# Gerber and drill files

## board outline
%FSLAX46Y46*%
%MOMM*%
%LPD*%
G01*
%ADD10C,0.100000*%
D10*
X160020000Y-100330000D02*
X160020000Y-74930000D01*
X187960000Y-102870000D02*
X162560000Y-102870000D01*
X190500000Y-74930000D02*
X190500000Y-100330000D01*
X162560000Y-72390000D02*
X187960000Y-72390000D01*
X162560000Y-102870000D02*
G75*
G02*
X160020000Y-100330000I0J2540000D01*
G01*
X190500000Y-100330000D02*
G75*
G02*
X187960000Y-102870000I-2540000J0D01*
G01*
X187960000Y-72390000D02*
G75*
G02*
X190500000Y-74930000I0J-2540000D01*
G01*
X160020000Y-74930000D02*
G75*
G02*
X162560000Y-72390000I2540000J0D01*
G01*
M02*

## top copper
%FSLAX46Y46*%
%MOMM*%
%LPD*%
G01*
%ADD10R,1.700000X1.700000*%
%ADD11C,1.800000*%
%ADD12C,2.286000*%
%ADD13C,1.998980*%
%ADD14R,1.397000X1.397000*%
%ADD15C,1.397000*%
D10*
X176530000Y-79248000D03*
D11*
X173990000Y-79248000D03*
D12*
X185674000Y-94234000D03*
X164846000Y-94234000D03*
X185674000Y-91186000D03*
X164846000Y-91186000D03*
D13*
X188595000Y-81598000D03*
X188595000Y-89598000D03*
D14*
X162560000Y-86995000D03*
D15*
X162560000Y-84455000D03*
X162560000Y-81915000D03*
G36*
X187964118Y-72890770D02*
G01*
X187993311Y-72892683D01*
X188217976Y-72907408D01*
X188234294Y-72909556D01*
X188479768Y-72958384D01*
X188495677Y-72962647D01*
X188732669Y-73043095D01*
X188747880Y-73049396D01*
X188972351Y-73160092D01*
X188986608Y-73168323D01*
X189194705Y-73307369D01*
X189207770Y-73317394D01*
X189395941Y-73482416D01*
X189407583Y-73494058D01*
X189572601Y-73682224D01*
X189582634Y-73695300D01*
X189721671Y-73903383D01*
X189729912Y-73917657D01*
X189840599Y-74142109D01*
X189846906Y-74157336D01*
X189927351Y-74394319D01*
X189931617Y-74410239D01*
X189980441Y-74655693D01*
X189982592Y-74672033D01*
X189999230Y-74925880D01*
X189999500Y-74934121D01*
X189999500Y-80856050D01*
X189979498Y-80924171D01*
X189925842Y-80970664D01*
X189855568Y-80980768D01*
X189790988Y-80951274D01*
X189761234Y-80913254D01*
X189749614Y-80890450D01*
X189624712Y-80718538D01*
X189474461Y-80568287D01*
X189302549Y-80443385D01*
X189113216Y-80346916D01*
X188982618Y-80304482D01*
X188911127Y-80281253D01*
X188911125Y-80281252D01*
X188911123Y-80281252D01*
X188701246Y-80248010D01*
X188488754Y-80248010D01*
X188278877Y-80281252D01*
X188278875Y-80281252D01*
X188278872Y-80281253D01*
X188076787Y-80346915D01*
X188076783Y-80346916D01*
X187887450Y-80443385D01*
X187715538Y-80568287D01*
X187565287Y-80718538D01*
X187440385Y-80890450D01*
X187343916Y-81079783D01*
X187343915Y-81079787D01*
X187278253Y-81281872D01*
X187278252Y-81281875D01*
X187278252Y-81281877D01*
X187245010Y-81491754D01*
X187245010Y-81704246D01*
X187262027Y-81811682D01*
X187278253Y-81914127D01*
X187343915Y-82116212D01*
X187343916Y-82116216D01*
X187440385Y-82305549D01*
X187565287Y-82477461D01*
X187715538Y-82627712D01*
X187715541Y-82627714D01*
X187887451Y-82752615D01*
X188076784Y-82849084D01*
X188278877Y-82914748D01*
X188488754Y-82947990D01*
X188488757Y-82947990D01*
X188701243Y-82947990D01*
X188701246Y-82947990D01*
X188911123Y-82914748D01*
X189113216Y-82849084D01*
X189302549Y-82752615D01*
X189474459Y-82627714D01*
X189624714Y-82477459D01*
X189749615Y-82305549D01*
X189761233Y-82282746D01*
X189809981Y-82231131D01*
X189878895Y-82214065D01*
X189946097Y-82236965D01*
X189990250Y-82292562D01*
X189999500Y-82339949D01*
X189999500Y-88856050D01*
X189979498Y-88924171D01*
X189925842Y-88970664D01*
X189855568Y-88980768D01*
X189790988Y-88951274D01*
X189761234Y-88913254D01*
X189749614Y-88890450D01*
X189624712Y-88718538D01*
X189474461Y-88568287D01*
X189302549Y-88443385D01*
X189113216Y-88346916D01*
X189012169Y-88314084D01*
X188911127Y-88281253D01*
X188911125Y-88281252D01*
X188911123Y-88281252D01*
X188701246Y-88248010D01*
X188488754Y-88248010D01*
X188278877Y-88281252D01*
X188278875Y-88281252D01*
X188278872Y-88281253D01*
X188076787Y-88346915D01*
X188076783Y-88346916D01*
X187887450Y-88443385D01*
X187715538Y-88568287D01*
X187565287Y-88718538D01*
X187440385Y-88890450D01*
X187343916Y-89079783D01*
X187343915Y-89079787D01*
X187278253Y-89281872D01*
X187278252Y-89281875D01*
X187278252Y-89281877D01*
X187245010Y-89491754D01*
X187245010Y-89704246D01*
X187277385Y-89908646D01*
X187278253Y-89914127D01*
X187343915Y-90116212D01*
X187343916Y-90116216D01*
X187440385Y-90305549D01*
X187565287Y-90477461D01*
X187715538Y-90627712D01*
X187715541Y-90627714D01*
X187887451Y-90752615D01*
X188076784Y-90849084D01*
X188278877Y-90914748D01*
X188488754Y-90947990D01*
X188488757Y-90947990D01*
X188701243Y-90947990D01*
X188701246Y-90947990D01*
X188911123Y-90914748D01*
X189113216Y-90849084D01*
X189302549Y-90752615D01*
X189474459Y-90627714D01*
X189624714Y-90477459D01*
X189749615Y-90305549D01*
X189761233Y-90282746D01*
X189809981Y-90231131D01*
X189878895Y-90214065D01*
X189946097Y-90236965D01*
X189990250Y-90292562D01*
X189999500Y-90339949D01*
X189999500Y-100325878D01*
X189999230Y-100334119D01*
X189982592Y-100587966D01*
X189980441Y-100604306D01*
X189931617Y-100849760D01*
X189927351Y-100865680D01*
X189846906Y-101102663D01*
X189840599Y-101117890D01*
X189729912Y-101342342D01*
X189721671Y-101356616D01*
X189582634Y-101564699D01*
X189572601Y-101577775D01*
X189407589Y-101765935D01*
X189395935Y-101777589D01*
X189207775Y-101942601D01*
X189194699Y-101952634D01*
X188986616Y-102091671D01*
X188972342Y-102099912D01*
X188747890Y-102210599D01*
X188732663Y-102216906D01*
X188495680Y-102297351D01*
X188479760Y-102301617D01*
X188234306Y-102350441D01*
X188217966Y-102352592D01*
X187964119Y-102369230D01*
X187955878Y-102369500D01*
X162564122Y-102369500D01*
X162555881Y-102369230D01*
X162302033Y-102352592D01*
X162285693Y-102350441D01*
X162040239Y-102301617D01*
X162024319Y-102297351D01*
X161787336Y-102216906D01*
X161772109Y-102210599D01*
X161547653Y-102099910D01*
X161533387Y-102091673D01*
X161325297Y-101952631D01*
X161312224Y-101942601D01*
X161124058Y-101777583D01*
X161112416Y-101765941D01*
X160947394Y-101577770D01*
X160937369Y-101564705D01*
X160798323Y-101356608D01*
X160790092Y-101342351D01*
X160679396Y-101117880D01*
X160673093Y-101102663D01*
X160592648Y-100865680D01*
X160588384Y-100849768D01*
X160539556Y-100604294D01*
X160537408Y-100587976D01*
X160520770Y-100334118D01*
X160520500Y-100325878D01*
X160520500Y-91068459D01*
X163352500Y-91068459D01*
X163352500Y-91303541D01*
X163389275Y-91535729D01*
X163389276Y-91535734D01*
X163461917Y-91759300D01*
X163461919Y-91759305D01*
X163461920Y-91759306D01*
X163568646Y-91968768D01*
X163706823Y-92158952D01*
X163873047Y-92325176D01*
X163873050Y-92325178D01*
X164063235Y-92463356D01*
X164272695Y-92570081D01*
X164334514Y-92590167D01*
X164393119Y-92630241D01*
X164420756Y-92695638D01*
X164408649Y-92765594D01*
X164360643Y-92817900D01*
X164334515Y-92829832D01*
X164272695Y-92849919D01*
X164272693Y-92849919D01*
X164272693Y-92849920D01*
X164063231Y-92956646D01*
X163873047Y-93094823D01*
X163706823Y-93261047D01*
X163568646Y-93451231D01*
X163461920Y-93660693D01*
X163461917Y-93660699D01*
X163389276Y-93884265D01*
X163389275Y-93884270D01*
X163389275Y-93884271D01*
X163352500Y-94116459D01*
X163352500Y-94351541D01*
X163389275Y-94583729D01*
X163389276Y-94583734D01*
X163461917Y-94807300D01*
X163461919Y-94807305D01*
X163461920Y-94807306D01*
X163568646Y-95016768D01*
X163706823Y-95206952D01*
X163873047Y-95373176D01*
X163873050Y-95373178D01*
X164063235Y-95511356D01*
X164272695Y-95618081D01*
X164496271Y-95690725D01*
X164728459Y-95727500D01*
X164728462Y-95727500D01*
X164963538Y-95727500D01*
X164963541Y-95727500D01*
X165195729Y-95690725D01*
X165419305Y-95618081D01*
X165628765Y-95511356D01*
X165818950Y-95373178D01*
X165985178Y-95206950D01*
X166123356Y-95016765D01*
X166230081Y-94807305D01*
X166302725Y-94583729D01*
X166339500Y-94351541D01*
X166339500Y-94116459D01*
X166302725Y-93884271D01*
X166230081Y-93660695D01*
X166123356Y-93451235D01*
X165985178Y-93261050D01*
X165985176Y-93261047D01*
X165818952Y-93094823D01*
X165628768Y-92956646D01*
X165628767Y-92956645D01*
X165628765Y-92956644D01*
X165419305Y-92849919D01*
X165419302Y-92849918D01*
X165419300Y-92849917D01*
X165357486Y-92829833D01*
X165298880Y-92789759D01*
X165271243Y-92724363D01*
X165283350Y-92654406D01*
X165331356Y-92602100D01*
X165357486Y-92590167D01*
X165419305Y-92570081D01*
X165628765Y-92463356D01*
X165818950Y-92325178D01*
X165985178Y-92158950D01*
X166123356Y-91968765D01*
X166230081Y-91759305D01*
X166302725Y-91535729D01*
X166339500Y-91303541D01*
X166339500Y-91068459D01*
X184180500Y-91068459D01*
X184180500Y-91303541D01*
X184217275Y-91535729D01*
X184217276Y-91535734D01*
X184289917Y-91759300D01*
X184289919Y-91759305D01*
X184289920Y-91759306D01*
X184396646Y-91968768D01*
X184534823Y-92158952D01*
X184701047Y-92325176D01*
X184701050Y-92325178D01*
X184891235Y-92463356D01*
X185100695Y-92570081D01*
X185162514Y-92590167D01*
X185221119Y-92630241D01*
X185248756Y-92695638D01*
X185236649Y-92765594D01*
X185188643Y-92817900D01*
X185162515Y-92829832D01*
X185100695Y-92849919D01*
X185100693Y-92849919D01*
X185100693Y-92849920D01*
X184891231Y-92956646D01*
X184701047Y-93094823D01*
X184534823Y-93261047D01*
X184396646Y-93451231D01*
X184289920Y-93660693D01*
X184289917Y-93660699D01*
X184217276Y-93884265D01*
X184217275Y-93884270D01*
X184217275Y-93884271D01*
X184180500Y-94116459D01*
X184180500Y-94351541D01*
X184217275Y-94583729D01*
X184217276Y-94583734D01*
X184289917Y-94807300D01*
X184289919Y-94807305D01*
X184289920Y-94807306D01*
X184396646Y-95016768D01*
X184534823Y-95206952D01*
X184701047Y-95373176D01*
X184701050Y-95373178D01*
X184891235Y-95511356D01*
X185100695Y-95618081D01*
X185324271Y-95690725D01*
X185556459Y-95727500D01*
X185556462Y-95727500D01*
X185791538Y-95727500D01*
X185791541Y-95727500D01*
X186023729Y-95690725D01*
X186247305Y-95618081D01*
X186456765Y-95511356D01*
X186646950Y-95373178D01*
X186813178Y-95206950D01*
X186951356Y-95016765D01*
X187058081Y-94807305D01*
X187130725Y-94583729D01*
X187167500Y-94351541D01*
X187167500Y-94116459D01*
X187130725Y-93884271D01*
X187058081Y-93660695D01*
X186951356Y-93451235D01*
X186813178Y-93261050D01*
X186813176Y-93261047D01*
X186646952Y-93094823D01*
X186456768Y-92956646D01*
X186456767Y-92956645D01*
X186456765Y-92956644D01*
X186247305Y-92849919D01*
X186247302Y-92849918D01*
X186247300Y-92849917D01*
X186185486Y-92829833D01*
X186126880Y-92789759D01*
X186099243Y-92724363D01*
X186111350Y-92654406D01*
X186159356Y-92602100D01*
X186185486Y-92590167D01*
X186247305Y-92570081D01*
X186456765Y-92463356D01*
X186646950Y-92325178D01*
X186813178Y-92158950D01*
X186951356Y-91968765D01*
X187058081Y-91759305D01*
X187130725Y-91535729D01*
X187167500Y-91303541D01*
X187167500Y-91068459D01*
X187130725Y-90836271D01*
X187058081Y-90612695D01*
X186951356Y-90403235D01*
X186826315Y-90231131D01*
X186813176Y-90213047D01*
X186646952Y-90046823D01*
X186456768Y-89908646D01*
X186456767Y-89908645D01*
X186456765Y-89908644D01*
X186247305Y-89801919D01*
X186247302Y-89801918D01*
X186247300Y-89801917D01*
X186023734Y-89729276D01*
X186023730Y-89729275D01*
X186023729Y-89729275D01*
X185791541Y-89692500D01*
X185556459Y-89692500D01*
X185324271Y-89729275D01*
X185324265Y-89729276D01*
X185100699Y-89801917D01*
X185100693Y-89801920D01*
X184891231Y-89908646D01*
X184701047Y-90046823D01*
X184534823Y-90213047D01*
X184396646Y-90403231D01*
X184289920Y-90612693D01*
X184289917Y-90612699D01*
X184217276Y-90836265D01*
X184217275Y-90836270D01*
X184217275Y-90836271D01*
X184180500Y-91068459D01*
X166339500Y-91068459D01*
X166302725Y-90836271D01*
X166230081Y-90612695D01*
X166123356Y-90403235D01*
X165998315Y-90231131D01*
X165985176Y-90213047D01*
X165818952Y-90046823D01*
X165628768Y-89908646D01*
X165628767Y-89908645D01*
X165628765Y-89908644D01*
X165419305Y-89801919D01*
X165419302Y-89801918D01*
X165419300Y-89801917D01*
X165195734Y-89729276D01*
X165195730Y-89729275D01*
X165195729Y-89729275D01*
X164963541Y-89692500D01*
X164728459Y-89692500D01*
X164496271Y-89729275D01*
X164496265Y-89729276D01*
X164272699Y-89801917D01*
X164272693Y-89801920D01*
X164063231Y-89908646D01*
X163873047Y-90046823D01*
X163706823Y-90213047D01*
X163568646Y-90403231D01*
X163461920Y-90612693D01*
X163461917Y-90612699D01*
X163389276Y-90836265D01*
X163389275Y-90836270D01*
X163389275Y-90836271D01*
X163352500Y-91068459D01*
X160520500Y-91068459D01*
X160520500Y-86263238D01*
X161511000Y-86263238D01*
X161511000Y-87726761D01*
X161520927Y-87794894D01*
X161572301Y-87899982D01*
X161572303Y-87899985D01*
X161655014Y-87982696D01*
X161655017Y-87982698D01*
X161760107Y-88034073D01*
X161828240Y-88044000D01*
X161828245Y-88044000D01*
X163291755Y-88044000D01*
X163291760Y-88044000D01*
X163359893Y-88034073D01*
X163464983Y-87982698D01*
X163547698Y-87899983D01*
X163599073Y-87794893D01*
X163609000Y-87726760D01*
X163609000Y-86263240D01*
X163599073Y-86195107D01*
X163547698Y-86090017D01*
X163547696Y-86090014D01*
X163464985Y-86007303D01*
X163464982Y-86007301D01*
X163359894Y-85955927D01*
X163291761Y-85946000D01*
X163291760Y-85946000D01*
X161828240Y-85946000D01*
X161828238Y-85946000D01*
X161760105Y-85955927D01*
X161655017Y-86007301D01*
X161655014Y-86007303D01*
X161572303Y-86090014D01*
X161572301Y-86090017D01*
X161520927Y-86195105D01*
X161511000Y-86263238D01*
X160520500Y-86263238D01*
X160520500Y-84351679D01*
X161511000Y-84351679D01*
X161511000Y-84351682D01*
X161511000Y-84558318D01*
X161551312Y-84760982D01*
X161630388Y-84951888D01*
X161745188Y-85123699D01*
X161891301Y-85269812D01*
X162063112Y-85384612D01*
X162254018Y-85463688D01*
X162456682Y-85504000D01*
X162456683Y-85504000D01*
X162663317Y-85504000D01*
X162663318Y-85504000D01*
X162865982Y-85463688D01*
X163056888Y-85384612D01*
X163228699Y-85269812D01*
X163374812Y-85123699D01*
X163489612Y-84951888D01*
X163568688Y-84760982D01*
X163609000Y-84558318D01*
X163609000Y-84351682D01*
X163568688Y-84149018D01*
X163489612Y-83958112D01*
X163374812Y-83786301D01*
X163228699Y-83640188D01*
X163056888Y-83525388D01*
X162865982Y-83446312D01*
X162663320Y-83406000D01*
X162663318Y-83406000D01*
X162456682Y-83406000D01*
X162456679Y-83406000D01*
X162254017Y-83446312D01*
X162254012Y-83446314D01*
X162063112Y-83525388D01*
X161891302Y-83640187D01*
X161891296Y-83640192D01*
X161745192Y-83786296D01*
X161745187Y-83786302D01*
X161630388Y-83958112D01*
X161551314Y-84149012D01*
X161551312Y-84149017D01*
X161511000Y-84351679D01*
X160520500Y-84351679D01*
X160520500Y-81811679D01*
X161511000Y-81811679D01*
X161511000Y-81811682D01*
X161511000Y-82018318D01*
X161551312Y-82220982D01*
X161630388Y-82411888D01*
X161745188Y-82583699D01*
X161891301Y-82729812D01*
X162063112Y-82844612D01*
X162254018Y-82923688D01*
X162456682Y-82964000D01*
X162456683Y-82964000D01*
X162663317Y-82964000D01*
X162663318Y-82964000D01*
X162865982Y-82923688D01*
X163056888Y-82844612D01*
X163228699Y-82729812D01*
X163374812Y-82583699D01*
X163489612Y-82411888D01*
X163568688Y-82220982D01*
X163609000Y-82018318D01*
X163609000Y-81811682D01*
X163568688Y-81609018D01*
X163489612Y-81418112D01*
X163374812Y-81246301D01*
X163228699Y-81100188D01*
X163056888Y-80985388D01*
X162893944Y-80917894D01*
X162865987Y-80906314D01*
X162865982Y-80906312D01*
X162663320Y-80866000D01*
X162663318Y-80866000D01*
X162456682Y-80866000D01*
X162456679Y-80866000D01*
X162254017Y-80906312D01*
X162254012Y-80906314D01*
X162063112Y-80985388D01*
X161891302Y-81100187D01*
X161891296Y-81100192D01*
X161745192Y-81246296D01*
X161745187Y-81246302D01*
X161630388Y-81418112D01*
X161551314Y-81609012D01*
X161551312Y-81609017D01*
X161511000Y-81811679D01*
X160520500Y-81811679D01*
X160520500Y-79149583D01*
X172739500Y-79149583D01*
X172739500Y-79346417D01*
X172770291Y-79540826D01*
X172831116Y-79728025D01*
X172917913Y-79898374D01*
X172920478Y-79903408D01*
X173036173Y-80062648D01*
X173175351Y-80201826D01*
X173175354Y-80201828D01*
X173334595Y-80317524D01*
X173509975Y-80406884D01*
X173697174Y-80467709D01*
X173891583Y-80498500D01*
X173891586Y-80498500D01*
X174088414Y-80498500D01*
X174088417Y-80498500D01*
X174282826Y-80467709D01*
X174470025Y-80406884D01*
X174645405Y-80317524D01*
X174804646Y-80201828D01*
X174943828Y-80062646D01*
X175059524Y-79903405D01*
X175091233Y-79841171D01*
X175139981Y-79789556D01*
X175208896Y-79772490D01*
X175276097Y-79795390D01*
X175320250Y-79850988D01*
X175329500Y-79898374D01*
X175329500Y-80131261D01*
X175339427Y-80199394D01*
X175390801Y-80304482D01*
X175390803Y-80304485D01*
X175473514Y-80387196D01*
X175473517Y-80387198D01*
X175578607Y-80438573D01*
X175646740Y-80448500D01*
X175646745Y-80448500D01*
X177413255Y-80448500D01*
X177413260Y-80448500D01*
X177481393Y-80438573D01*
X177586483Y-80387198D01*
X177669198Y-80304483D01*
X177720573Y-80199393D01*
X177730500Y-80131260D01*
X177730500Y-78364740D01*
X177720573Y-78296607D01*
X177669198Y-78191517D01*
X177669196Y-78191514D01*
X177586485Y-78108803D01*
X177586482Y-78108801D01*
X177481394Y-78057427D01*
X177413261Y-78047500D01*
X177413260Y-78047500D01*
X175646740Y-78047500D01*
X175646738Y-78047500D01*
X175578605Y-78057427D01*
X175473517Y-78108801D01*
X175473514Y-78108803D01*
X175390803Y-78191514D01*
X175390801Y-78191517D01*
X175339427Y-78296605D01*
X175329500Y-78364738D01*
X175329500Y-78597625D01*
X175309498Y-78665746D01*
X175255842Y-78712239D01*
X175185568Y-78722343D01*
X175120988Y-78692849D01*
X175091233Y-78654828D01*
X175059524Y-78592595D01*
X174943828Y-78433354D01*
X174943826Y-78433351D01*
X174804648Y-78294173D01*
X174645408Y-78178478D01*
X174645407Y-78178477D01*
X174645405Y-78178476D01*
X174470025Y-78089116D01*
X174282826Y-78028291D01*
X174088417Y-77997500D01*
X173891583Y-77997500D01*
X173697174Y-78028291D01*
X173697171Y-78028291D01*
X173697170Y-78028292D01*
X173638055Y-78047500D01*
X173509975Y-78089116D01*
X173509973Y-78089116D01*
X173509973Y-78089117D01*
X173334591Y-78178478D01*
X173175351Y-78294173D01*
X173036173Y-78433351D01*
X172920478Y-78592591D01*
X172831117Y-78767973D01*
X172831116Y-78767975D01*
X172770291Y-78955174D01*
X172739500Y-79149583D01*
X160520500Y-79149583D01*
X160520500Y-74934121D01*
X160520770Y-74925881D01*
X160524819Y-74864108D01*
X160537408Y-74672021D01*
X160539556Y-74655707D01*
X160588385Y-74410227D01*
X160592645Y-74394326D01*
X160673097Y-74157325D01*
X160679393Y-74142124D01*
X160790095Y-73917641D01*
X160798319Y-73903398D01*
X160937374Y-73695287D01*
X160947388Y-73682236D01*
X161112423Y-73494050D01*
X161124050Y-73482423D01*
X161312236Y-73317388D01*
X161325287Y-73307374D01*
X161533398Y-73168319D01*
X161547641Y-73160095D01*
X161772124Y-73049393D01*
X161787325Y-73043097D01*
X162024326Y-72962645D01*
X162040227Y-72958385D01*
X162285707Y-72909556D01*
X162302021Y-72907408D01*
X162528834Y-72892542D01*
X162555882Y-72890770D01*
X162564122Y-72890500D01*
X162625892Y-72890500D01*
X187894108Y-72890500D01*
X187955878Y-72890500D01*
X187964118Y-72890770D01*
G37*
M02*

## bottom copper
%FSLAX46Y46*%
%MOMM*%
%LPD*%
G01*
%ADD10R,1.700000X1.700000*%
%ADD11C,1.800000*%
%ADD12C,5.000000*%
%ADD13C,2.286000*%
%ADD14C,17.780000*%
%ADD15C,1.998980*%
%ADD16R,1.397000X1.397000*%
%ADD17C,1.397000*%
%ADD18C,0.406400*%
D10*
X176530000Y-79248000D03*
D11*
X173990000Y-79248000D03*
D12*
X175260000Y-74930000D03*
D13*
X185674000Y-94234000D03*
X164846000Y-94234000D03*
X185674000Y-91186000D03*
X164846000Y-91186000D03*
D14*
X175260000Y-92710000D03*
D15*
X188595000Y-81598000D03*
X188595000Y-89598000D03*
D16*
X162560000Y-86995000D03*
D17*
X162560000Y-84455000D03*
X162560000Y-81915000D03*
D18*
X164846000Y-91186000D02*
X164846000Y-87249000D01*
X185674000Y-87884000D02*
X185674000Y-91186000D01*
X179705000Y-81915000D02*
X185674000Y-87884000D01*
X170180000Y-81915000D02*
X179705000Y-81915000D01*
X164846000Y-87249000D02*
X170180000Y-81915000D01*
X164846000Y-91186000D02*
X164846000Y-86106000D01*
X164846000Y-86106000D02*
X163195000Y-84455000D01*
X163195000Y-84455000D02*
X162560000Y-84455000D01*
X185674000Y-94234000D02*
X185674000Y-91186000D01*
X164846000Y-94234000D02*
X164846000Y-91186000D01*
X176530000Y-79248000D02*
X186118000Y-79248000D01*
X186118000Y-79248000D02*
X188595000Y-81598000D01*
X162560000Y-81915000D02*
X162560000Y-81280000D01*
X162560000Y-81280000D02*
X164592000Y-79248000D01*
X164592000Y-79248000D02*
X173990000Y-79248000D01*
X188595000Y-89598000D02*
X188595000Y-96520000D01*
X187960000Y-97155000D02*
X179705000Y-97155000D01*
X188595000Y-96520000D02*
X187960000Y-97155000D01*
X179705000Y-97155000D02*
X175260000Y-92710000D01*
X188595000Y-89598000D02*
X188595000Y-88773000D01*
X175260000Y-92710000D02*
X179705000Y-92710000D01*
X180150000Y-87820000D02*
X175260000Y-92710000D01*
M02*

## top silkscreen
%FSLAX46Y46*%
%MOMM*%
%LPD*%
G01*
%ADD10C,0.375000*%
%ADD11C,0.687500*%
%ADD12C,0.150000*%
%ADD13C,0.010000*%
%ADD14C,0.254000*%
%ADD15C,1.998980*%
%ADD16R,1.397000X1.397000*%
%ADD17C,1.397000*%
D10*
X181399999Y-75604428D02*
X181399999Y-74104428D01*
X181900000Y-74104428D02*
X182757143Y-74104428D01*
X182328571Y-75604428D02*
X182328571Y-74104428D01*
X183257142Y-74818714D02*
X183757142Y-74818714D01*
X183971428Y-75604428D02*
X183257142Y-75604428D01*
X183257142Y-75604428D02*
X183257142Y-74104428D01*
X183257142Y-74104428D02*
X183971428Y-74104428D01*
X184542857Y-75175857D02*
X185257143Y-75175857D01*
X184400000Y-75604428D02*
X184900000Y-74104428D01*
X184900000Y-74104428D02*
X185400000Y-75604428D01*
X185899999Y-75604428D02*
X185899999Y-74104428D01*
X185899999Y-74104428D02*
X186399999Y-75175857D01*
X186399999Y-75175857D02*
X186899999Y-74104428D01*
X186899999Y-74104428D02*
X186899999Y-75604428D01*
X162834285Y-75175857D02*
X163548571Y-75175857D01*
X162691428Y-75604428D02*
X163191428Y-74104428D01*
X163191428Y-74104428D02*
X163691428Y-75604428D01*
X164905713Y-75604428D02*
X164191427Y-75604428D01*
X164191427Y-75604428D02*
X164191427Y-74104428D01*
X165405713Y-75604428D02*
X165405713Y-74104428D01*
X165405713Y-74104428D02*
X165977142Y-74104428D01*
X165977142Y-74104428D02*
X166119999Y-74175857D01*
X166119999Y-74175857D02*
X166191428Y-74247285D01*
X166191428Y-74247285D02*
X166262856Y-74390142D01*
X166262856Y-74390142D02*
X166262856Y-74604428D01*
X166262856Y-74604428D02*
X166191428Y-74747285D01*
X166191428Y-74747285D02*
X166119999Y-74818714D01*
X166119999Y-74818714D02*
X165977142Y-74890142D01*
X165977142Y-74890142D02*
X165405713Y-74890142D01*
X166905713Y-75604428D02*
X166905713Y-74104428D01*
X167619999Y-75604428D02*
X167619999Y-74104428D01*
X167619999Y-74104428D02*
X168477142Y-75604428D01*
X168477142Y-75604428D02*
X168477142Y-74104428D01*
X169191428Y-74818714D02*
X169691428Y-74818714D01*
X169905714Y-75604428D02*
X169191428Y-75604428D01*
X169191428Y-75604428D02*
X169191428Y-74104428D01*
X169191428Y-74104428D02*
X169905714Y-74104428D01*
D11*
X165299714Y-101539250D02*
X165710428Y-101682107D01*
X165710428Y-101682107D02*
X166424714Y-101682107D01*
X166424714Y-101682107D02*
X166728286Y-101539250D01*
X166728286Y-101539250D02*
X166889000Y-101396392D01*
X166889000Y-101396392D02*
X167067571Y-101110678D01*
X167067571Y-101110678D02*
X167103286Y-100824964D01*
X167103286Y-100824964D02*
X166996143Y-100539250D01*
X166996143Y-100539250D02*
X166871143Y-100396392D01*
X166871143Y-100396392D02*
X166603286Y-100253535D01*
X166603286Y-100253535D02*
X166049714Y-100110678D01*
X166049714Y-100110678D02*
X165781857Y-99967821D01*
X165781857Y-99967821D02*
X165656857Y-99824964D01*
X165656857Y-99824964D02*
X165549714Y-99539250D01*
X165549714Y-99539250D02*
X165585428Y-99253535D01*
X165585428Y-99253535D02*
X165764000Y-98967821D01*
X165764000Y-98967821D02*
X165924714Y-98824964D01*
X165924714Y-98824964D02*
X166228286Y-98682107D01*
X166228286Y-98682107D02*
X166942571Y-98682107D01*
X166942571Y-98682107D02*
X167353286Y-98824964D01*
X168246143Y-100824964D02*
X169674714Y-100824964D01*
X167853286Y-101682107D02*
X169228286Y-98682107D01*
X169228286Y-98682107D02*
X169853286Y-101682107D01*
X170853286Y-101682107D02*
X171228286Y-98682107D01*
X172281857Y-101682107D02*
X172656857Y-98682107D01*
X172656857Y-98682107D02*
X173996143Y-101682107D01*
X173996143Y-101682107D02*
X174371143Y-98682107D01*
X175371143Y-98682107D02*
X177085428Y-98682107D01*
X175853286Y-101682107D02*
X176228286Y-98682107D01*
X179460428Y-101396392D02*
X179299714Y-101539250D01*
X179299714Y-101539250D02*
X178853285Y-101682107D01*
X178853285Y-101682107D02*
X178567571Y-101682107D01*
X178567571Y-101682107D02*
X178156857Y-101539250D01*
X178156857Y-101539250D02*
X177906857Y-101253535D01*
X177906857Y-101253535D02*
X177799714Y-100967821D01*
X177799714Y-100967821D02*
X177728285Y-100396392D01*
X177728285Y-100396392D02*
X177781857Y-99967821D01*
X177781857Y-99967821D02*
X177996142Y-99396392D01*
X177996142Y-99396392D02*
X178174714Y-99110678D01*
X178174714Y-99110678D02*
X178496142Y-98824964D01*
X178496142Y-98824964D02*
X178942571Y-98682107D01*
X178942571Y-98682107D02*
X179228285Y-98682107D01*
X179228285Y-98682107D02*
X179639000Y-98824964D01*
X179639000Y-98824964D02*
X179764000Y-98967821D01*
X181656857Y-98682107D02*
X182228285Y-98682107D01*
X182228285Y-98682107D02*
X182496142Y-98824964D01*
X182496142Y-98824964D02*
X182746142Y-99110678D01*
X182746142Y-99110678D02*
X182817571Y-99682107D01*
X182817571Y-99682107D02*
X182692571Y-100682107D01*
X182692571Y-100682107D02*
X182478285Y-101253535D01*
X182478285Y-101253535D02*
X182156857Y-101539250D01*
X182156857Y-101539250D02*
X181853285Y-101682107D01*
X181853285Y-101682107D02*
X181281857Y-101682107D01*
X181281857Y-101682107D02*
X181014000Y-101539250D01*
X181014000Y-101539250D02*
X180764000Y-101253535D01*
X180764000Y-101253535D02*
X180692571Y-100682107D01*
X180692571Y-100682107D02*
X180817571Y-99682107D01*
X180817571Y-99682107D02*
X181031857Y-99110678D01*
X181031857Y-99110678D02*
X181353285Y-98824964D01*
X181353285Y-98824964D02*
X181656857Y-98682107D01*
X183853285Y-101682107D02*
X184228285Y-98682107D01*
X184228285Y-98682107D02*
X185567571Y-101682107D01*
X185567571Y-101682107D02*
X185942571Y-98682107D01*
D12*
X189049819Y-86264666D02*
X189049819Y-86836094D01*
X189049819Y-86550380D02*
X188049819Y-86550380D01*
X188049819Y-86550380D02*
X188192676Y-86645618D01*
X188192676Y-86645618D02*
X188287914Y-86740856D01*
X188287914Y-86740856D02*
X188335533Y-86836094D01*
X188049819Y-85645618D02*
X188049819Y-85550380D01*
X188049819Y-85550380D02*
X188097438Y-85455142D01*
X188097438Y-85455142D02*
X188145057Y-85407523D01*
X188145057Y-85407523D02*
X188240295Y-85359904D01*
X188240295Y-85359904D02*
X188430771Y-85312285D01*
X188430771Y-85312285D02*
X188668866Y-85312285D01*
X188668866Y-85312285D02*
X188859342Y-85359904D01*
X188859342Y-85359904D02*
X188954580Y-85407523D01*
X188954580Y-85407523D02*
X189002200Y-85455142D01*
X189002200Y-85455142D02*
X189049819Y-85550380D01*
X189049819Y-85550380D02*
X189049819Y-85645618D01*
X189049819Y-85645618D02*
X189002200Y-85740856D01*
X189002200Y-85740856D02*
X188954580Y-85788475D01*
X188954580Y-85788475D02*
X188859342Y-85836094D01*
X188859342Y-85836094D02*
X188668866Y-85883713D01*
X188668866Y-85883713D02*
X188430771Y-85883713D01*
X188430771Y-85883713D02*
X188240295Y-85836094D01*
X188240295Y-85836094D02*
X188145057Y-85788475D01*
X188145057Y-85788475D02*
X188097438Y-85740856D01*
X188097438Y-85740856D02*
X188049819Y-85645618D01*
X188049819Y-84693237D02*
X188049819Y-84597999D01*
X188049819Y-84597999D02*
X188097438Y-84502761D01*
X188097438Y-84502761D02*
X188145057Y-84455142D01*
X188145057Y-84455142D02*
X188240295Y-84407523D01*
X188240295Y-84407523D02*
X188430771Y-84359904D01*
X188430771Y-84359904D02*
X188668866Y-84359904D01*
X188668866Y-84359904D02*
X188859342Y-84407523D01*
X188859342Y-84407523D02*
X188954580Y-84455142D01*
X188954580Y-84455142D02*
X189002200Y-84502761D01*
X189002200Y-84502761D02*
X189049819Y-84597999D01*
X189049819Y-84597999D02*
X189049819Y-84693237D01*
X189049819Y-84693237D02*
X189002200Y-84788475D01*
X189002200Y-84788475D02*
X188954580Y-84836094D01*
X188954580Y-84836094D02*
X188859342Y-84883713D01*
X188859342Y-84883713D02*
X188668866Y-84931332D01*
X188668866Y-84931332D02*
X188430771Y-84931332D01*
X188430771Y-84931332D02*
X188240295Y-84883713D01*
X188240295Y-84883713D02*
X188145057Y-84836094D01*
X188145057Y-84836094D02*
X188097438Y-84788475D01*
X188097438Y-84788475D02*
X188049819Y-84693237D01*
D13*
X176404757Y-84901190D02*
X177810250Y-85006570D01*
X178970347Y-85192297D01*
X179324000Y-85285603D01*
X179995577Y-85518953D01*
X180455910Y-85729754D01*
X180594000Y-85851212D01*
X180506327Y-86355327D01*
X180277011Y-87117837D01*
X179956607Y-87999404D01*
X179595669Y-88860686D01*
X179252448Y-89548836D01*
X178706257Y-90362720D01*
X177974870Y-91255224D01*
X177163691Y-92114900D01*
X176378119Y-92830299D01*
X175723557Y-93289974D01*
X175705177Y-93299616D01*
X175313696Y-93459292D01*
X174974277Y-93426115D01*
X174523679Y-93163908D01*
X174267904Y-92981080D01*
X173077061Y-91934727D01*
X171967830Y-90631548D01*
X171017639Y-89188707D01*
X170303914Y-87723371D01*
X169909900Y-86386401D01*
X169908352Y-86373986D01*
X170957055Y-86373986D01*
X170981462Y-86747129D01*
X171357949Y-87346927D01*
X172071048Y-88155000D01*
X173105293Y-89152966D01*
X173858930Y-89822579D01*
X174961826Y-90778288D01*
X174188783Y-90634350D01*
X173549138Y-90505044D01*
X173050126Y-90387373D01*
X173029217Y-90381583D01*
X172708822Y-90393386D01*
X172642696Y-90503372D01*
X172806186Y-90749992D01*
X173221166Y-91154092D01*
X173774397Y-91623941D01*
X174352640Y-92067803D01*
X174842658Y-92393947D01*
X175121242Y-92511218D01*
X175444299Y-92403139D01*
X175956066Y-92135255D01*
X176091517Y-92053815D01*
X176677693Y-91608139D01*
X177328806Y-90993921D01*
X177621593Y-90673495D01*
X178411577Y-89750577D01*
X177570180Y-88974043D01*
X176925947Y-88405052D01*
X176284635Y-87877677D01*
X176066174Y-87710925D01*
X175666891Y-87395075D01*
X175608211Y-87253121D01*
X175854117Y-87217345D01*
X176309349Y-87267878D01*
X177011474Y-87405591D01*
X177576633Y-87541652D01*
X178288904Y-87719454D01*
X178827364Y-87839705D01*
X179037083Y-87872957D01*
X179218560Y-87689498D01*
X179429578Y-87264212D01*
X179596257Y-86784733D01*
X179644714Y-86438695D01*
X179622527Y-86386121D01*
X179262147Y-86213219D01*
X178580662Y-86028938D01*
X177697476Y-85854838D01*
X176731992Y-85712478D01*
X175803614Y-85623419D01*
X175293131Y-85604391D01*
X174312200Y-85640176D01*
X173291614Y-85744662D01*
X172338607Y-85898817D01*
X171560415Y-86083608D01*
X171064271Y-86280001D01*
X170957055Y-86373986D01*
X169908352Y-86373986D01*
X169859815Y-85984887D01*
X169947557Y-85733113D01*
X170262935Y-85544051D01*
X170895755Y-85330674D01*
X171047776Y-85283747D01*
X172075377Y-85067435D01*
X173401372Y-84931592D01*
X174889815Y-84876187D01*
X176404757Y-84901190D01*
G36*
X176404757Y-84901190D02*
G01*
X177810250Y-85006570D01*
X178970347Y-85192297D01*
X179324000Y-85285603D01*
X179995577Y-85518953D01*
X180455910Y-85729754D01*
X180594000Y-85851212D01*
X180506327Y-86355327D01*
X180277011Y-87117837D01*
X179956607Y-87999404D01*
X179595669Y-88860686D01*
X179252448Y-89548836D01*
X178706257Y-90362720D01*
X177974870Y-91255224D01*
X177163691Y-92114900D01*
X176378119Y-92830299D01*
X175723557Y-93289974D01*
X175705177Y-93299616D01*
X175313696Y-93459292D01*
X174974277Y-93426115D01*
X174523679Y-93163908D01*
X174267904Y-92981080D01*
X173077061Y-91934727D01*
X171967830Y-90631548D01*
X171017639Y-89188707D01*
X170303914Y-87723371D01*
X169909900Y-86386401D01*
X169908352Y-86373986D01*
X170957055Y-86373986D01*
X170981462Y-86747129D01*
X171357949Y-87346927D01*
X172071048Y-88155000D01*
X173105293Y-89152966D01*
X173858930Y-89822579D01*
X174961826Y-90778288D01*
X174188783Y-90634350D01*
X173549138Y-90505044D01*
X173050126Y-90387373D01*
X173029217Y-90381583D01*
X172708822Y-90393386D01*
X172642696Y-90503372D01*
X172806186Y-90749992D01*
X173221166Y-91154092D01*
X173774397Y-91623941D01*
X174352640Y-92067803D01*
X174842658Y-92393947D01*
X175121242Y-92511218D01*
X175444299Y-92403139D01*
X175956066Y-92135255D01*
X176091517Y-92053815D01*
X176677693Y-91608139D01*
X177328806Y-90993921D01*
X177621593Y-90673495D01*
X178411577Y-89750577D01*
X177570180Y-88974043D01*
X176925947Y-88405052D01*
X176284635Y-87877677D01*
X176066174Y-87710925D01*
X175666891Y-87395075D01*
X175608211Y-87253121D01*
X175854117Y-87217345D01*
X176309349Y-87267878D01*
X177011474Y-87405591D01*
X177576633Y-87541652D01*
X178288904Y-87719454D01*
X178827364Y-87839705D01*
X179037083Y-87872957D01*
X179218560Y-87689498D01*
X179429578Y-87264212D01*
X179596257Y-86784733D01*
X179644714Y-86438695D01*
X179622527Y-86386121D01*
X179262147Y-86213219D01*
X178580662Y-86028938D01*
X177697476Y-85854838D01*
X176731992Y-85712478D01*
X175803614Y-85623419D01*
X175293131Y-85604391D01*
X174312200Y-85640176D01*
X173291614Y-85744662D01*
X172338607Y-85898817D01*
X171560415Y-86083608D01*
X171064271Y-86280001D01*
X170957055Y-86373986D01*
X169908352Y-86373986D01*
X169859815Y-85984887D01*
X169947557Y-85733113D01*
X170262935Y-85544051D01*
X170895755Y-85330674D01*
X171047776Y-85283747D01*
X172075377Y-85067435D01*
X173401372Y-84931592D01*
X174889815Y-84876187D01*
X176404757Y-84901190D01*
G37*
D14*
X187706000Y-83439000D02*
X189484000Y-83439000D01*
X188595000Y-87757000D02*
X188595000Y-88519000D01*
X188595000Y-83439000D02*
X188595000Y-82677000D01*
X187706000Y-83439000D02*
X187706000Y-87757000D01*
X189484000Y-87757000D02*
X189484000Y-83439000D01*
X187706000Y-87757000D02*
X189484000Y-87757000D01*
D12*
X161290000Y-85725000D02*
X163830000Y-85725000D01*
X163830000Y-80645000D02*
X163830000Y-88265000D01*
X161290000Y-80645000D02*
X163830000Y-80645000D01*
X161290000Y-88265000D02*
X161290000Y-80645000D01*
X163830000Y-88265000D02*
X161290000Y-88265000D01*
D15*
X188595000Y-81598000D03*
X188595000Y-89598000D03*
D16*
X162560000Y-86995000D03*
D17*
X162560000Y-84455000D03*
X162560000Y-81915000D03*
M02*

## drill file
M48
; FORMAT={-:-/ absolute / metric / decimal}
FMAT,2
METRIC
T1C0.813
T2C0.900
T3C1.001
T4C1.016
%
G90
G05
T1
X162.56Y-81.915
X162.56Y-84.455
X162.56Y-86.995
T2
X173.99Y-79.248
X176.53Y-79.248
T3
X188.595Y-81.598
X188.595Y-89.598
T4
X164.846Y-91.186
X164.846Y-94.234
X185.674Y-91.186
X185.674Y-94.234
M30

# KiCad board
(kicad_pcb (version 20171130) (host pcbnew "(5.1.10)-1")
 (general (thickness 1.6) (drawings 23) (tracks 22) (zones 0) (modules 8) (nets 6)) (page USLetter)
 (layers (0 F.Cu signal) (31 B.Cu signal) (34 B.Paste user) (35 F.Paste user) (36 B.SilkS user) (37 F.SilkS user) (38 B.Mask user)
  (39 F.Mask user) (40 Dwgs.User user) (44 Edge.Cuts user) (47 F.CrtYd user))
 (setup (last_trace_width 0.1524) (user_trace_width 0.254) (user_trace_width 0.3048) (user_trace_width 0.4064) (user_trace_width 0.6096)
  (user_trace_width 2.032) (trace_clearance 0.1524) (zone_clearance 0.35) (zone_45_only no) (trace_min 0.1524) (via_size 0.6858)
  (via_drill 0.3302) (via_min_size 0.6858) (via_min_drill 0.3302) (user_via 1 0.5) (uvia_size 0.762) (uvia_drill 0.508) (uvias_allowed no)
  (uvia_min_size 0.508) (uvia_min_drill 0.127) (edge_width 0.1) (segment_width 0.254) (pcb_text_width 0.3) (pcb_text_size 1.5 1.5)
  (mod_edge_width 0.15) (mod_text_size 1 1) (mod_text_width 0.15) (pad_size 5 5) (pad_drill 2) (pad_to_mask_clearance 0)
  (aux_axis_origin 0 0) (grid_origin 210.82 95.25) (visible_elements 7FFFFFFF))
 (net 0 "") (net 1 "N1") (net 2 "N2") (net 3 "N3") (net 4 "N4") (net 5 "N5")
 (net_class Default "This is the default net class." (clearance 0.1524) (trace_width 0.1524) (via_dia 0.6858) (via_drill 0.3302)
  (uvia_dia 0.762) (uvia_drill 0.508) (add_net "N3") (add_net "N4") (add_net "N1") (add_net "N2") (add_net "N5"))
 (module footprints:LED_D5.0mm (layer F.Cu) (at 176.53 79.248 180)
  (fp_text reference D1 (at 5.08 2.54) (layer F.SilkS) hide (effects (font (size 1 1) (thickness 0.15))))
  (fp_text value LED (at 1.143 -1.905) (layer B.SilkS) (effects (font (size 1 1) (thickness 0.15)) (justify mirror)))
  (pad 1 thru_hole rect (at 0 0 180) (size 1.7 1.7) (drill 0.9) (layers B.Cu B.Mask) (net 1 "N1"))
  (pad 2 thru_hole circle (at 2.54 0 180) (size 1.8 1.8) (drill 0.9) (layers B.Cu B.Mask) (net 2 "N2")))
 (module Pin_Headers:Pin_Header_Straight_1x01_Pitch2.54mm (layer F.Cu) (at 175.26 74.93)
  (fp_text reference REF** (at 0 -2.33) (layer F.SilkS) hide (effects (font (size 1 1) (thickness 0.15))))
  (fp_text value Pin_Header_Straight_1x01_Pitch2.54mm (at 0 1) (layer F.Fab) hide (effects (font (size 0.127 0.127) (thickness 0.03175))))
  (pad 1 smd circle (at 0 0) (size 5 5) (layers B.Cu B.Paste B.Mask)))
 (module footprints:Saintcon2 (layer F.Cu) (at 175.514 86.106)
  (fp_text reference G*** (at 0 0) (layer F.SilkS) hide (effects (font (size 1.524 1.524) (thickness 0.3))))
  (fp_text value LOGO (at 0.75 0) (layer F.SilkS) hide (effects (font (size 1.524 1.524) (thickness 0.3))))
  (fp_poly
   (pts (xy 0.890757 -1.20481) (xy 2.29625 -1.09943) (xy 3.456347 -0.913703) (xy 3.81 -0.820397) (xy 4.481577 -0.587047)
    (xy 4.94191 -0.376246) (xy 5.08 -0.254788) (xy 4.992327 0.249327) (xy 4.763011 1.011837) (xy 4.442607 1.893404) (xy 4.081669 2.754686)
    (xy 3.738448 3.442836) (xy 3.192257 4.25672) (xy 2.46087 5.149224) (xy 1.649691 6.0089) (xy 0.864119 6.724299) (xy 0.209557 7.183974)
    (xy 0.191177 7.193616) (xy -0.200304 7.353292) (xy -0.539723 7.320115) (xy -0.990321 7.057908) (xy -1.246096 6.87508)
    (xy -2.436939 5.828727) (xy -3.54617 4.525548) (xy -4.496361 3.082707) (xy -5.210086 1.617371) (xy -5.6041 0.280401)
    (xy -5.605648 0.267986) (xy -4.556945 0.267986) (xy -4.532538 0.641129) (xy -4.156051 1.240927) (xy -3.442952 2.049)
    (xy -2.408707 3.046966) (xy -1.65507 3.716579) (xy -0.552174 4.672288) (xy -1.325217 4.52835) (xy -1.964862 4.399044)
    (xy -2.463874 4.281373) (xy -2.484783 4.275583) (xy -2.805178 4.287386) (xy -2.871304 4.397372) (xy -2.707814 4.643992)
    (xy -2.292834 5.048092) (xy -1.739603 5.517941) (xy -1.16136 5.961803) (xy -0.671342 6.287947) (xy -0.392758 6.405218)
    (xy -0.069701 6.297139) (xy 0.442066 6.029255) (xy 0.577517 5.947815) (xy 1.163693 5.502139) (xy 1.814806 4.887921)
    (xy 2.107593 4.567495) (xy 2.897577 3.644577) (xy 2.05618 2.868043) (xy 1.411947 2.299052) (xy 0.770635 1.771677) (xy 0.552174 1.604925)
    (xy 0.152891 1.289075) (xy 0.094211 1.147121) (xy 0.340117 1.111345) (xy 0.795349 1.161878) (xy 1.497474 1.299591)
    (xy 2.062633 1.435652) (xy 2.774904 1.613454) (xy 3.313364 1.733705) (xy 3.523083 1.766957) (xy 3.70456 1.583498) (xy 3.915578 1.158212)
    (xy 4.082257 0.678733) (xy 4.130714 0.332695) (xy 4.108527 0.280121) (xy 3.748147 0.107219) (xy 3.066662 -0.077062)
    (xy 2.183476 -0.251162) (xy 1.217992 -0.393522) (xy 0.289614 -0.482581) (xy -0.220869 -0.501609) (xy -1.2018 -0.465824)
    (xy -2.222386 -0.361338) (xy -3.175393 -0.207183) (xy -3.953585 -0.022392) (xy -4.449729 0.174001) (xy -4.556945 0.267986)
    (xy -5.605648 0.267986) (xy -5.654185 -0.121113) (xy -5.566443 -0.372887) (xy -5.251065 -0.561949) (xy -4.618245 -0.775326)
    (xy -4.466224 -0.822253) (xy -3.438623 -1.038565) (xy -2.112628 -1.174408) (xy -0.624185 -1.229813) (xy 0.890757 -1.20481))
   (layer F.SilkS) (width 0.01)))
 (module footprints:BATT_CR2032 (layer B.Cu) (at 175.26 92.71 180)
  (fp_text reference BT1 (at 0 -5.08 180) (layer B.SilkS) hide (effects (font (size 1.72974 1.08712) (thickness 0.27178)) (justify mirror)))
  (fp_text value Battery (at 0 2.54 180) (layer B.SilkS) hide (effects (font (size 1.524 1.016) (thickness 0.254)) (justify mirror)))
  (pad 1 thru_hole circle (at -10.414 -1.524 180) (size 2.286 2.286) (drill 1.016) (layers *.Cu *.Mask B.SilkS) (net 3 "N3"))
  (pad 1 thru_hole circle (at 10.414 -1.524 180) (size 2.286 2.286) (drill 1.016) (layers *.Cu *.Mask B.SilkS) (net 3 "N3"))
  (pad 1 thru_hole circle (at -10.414 1.524 180) (size 2.286 2.286) (drill 1.016) (layers *.Cu *.Mask B.SilkS) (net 3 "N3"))
  (pad 1 thru_hole circle (at 10.414 1.524 180) (size 2.286 2.286) (drill 1.016) (layers *.Cu *.Mask B.SilkS) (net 3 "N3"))
  (pad 2 smd circle (at 0 0 180) (size 17.78 17.78) (layers B.Cu B.Paste B.Mask) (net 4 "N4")))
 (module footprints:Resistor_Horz (layer F.Cu) (at 188.595 85.598 270)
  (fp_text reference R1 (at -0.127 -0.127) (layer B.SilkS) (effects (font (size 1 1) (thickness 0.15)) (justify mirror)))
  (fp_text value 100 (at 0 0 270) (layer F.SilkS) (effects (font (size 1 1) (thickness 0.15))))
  (fp_line (start -2.159 0.889) (end -2.159 -0.889) (layer F.SilkS) (width 0.254))
  (fp_line (start 2.159 0) (end 2.921 0) (layer F.SilkS) (width 0.254))
  (fp_line (start -2.159 0) (end -2.921 0) (layer F.SilkS) (width 0.254))
  (fp_line (start -2.159 0.889) (end 2.159 0.889) (layer F.SilkS) (width 0.254))
  (fp_line (start 2.159 -0.889) (end -2.159 -0.889) (layer F.SilkS) (width 0.254))
  (fp_line (start 2.159 0.889) (end 2.159 -0.889) (layer F.SilkS) (width 0.254))
  (pad 1 thru_hole circle (at -4 0 270) (size 1.99898 1.99898) (drill 1.00076) (layers *.Cu *.SilkS *.Mask) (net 1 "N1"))
  (pad 2 thru_hole circle (at 4 0 270) (size 1.99898 1.99898) (drill 1.00076) (layers *.Cu *.SilkS *.Mask) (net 4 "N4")))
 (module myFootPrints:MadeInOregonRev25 (layer F.Cu) (at 167.64 76.454)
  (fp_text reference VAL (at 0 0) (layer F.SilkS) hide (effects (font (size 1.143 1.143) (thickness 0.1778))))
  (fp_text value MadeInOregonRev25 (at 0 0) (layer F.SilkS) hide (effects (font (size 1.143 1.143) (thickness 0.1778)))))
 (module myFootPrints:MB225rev (layer F.Cu) (at 184.15 76.2)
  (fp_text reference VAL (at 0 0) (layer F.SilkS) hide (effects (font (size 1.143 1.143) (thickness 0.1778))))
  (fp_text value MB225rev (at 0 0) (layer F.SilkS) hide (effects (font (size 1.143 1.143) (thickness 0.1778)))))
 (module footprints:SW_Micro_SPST (layer F.Cu) (at 162.56 84.455 90)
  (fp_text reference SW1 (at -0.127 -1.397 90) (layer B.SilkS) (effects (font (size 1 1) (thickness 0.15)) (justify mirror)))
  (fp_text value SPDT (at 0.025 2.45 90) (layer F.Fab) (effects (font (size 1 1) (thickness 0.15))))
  (fp_line (start -1.27 -1.27) (end -1.27 1.27) (layer F.SilkS) (width 0.15))
  (fp_line (start 3.81 1.27) (end -3.81 1.27) (layer F.SilkS) (width 0.15))
  (fp_line (start 3.81 -1.27) (end 3.81 1.27) (layer F.SilkS) (width 0.15))
  (fp_line (start -3.81 -1.27) (end 3.81 -1.27) (layer F.SilkS) (width 0.15))
  (fp_line (start -3.81 1.27) (end -3.81 -1.27) (layer F.SilkS) (width 0.15))
  (pad 1 thru_hole rect (at -2.54 0 90) (size 1.397 1.397) (drill 0.8128) (layers *.Cu *.Mask F.SilkS) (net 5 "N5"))
  (pad 2 thru_hole circle (at 0 0 90) (size 1.397 1.397) (drill 0.8128) (layers *.Cu *.Mask F.SilkS) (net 3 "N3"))
  (pad 3 thru_hole circle (at 2.54 0 90) (size 1.397 1.397) (drill 0.8128) (layers *.Cu *.Mask F.SilkS) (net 2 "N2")))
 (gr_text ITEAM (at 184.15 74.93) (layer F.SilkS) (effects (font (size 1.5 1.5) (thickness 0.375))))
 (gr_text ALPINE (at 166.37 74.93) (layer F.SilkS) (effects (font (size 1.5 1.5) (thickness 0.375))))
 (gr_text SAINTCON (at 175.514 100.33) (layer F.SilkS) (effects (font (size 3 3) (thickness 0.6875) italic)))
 (gr_line (start 160.02 100.33) (end 160.02 74.93) (angle 90) (layer Edge.Cuts) (width 0.1))
 (gr_line (start 187.96 102.87) (end 162.56 102.87) (angle 90) (layer Edge.Cuts) (width 0.1))
 (gr_line (start 190.5 74.93) (end 190.5 100.33) (angle 90) (layer Edge.Cuts) (width 0.1))
 (gr_line (start 162.56 72.39) (end 187.96 72.39) (angle 90) (layer Edge.Cuts) (width 0.1))
 (gr_arc (start 162.56 100.33) (end 162.56 102.87) (angle 90) (layer Edge.Cuts) (width 0.1))
 (gr_arc (start 187.96 100.33) (end 190.5 100.33) (angle 90) (layer Edge.Cuts) (width 0.1))
 (gr_arc (start 187.96 74.93) (end 187.96 72.39) (angle 90) (layer Edge.Cuts) (width 0.1))
 (gr_arc (start 162.56 74.93) (end 160.02 74.93) (angle 90) (layer Edge.Cuts) (width 0.1))
 (segment (start 164.846 91.186) (end 164.846 87.249) (width 0.4064) (layer B.Cu) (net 3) (status 10))
 (segment (start 185.674 87.884) (end 185.674 91.186) (width 0.4064) (layer B.Cu) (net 3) (status 20))
 (segment (start 179.705 81.915) (end 185.674 87.884) (width 0.4064) (layer B.Cu) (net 3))
 (segment (start 170.18 81.915) (end 179.705 81.915) (width 0.4064) (layer B.Cu) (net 3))
 (segment (start 164.846 87.249) (end 170.18 81.915) (width 0.4064) (layer B.Cu) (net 3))
 (segment (start 164.846 91.186) (end 164.846 86.106) (width 0.4064) (layer B.Cu) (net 3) (status 10))
 (segment (start 164.846 86.106) (end 163.195 84.455) (width 0.4064) (layer B.Cu) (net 3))
 (segment (start 163.195 84.455) (end 162.56 84.455) (width 0.4064) (layer B.Cu) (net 3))
 (segment (start 185.674 94.234) (end 185.674 91.186) (width 0.4064) (layer B.Cu) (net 3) (status 30))
 (segment (start 164.846 94.234) (end 164.846 91.186) (width 0.4064) (layer B.Cu) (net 3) (status 30))
 (segment (start 176.53 79.248) (end 186.118 79.248) (width 0.4064) (layer B.Cu) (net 1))
 (segment (start 186.118 79.248) (end 188.595 81.598) (width 0.4064) (layer B.Cu) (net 1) (status 20))
 (segment (start 162.56 81.915) (end 162.56 81.28) (width 0.4064) (layer B.Cu) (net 2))
 (segment (start 162.56 81.28) (end 164.592 79.248) (width 0.4064) (layer B.Cu) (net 2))
 (segment (start 164.592 79.248) (end 173.99 79.248) (width 0.4064) (layer B.Cu) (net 2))
 (segment (start 188.595 89.598) (end 188.595 96.52) (width 0.4064) (layer B.Cu) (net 4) (status 10))
 (segment (start 187.96 97.155) (end 179.705 97.155) (width 0.4064) (layer B.Cu) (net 4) (status 20))
 (segment (start 188.595 96.52) (end 187.96 97.155) (width 0.4064) (layer B.Cu) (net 4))
 (segment (start 179.705 97.155) (end 175.26 92.71) (width 0.4064) (layer B.Cu) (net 4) (status 30))
 (segment (start 188.595 89.598) (end 188.595 88.773) (width 0.4064) (layer B.Cu) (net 4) (status 30))
 (segment (start 175.26 92.71) (end 179.705 92.71) (width 0.4064) (layer B.Cu) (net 4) (status 30))
 (segment (start 180.15 87.82) (end 175.26 92.71) (width 0.4064) (layer B.Cu) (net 4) (status 30))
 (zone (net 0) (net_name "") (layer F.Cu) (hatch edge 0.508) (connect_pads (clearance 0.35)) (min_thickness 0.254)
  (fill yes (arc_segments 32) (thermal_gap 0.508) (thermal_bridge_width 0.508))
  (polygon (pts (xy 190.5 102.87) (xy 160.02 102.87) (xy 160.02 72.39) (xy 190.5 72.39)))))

